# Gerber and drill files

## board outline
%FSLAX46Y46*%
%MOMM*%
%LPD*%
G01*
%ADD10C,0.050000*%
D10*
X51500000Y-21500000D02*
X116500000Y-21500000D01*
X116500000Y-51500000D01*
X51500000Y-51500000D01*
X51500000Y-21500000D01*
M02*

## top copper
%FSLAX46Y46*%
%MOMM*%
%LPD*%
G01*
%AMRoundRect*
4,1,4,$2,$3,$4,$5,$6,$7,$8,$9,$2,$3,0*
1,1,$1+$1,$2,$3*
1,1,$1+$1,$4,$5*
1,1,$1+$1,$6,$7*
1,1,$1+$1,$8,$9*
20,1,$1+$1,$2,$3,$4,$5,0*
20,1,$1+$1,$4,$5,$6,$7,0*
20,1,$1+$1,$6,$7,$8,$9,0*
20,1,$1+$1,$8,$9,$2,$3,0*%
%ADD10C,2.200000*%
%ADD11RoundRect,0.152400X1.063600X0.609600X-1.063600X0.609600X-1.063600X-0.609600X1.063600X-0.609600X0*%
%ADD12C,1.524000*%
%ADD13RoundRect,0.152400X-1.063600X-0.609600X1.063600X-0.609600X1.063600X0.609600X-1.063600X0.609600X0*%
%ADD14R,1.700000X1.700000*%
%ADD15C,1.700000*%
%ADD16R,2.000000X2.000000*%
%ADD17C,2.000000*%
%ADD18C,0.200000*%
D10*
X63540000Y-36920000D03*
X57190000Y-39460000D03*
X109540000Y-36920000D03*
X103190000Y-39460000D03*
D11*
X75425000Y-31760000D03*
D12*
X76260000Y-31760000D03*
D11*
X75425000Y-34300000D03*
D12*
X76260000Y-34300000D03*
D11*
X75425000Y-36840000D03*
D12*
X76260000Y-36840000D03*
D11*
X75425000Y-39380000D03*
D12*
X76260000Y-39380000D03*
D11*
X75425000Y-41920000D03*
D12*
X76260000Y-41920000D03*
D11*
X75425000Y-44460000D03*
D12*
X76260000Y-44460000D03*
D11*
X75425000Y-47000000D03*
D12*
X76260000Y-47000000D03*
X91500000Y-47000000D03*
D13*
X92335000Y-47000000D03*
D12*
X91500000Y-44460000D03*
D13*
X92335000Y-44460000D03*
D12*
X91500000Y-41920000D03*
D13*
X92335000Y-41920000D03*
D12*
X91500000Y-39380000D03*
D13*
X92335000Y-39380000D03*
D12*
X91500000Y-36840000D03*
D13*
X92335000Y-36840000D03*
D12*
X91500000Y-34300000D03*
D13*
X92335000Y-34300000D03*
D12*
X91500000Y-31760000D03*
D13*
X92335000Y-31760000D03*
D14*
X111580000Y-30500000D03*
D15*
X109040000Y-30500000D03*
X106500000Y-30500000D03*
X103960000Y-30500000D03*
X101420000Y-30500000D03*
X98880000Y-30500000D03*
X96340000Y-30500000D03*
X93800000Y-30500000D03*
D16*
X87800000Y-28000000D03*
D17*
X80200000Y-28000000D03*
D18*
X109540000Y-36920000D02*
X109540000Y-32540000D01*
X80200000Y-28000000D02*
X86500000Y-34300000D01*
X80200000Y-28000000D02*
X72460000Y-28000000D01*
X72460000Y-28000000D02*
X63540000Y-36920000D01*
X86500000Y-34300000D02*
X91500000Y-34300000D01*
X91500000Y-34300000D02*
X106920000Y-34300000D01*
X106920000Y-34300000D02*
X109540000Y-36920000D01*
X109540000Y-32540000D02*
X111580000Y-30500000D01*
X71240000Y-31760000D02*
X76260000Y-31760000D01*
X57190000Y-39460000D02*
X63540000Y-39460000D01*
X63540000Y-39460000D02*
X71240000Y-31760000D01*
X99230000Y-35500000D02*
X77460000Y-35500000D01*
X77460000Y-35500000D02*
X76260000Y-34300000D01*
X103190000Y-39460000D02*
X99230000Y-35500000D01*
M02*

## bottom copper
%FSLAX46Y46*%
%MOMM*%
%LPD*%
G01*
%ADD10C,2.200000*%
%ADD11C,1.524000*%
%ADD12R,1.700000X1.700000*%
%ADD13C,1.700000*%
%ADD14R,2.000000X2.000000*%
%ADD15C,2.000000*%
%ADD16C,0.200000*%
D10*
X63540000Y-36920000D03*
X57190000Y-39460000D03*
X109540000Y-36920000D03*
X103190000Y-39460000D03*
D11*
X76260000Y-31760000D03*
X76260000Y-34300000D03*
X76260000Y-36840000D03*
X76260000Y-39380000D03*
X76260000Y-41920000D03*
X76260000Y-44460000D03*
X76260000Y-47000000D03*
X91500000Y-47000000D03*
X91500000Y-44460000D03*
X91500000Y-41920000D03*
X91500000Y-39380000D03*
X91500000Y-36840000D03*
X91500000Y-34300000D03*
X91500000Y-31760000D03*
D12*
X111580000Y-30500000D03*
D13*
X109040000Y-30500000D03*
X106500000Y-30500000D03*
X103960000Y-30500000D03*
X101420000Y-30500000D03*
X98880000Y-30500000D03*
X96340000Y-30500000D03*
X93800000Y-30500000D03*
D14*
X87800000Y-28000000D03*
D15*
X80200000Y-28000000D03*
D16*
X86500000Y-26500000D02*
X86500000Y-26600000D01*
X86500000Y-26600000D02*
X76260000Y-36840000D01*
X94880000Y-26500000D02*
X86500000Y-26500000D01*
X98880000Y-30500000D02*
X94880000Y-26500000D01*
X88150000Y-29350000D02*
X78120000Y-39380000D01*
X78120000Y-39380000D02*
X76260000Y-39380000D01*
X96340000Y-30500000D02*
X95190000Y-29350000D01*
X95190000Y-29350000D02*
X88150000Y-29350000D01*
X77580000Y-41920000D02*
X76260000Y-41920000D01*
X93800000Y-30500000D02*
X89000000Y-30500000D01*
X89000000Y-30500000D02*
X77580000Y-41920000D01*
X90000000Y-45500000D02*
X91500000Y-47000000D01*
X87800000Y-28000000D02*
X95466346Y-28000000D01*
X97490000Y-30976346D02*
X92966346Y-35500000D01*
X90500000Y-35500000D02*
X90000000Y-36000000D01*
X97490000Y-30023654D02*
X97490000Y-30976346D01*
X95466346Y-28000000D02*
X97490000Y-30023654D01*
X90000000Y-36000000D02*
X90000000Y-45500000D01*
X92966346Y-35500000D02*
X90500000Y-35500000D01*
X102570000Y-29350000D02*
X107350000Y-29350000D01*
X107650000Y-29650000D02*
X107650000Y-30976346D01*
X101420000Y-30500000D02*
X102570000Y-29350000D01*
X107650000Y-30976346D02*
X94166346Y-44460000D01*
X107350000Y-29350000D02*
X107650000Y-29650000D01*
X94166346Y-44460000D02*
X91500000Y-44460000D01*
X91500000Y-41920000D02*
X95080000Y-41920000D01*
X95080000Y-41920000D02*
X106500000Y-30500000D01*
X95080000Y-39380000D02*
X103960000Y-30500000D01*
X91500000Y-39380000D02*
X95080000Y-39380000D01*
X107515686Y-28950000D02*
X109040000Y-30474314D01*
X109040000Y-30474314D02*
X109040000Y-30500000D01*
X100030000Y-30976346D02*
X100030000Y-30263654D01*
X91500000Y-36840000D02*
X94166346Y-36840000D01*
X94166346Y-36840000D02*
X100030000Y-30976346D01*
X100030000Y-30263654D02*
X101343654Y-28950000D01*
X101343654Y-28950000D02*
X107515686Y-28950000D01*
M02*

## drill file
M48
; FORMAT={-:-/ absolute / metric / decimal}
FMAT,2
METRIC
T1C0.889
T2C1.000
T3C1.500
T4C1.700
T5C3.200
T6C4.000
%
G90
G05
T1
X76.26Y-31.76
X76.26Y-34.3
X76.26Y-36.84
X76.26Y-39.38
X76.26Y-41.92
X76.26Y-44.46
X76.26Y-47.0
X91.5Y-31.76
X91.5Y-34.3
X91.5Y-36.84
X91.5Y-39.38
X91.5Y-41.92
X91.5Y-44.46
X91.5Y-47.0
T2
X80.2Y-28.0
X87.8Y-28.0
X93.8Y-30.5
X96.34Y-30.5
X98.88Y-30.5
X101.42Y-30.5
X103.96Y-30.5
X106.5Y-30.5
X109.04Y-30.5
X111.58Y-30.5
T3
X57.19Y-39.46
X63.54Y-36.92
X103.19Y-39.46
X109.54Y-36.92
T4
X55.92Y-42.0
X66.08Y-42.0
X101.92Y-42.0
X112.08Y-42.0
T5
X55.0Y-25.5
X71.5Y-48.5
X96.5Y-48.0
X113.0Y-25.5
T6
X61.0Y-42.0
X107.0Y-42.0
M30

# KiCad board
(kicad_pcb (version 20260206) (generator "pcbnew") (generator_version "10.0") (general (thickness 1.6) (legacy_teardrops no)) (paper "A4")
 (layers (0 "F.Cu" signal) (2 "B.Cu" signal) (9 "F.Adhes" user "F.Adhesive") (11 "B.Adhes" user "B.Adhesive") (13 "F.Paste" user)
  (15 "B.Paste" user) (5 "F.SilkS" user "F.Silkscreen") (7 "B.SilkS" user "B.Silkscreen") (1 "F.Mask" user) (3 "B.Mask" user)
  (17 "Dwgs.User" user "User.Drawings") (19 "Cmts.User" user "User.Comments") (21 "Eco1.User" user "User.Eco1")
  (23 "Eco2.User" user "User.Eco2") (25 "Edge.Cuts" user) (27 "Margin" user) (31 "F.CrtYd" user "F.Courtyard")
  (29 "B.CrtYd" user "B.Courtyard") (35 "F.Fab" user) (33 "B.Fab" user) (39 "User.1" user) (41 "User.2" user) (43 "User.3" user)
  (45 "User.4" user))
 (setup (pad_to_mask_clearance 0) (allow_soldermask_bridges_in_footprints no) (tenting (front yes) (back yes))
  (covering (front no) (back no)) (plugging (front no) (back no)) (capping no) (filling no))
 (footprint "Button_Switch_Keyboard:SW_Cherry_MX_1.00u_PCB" (layer "F.Cu") (at 63.54 36.92)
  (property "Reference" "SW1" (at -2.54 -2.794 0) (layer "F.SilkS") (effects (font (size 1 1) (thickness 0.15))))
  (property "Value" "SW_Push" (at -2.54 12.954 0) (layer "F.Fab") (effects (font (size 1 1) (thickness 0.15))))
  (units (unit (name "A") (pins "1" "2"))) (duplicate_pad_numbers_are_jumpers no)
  (pad "" np_thru_hole circle (at -7.62 5.08) (size 1.7 1.7) (drill 1.7) (layers "*.Cu" "*.Mask"))
  (pad "" np_thru_hole circle (at -2.54 5.08) (size 4 4) (drill 4) (layers "*.Cu" "*.Mask"))
  (pad "" np_thru_hole circle (at 2.54 5.08) (size 1.7 1.7) (drill 1.7) (layers "*.Cu" "*.Mask"))
  (pad "1" thru_hole circle (at 0 0) (size 2.2 2.2) (drill 1.5) (layers "*.Cu" "*.Mask") (remove_unused_layers no) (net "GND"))
  (pad "2" thru_hole circle (at -6.35 2.54) (size 2.2 2.2) (drill 1.5) (layers "*.Cu" "*.Mask") (remove_unused_layers no)
   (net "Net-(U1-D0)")))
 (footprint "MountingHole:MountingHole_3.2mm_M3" (layer "F.Cu") (at 96.5 48)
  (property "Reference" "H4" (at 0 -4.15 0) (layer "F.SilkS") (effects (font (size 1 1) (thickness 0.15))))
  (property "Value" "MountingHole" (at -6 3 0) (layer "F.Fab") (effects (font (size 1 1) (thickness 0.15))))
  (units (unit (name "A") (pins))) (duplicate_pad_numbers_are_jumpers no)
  (pad "" np_thru_hole circle (at 0 0) (size 3.2 3.2) (drill 3.2) (layers "*.Cu" "*.Mask")))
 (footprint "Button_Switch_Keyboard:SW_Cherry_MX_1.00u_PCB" (layer "F.Cu") (at 109.54 36.92)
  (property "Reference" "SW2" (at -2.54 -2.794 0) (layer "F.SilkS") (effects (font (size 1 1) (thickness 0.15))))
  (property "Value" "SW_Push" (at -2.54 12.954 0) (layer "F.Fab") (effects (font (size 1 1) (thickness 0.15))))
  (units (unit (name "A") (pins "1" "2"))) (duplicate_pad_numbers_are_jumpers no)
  (pad "" np_thru_hole circle (at -7.62 5.08) (size 1.7 1.7) (drill 1.7) (layers "*.Cu" "*.Mask"))
  (pad "" np_thru_hole circle (at -2.54 5.08) (size 4 4) (drill 4) (layers "*.Cu" "*.Mask"))
  (pad "" np_thru_hole circle (at 2.54 5.08) (size 1.7 1.7) (drill 1.7) (layers "*.Cu" "*.Mask"))
  (pad "1" thru_hole circle (at 0 0) (size 2.2 2.2) (drill 1.5) (layers "*.Cu" "*.Mask") (remove_unused_layers no) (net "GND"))
  (pad "2" thru_hole circle (at -6.35 2.54) (size 2.2 2.2) (drill 1.5) (layers "*.Cu" "*.Mask") (remove_unused_layers no)
   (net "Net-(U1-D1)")))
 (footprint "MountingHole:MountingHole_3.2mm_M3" (layer "F.Cu") (at 71.5 48.5)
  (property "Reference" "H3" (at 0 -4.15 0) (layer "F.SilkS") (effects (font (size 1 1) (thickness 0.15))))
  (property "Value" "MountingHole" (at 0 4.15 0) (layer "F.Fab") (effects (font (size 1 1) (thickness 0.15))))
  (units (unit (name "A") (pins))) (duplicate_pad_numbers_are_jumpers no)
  (pad "" np_thru_hole circle (at 0 0) (size 3.2 3.2) (drill 3.2) (layers "*.Cu" "*.Mask")))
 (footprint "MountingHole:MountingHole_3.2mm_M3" (layer "F.Cu") (at 113 25.5)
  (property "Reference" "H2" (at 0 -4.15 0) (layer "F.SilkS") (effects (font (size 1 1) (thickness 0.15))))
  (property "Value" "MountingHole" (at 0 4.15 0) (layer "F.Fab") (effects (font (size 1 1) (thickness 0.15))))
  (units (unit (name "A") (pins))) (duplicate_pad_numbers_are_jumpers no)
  (pad "" np_thru_hole circle (at 0 0) (size 3.2 3.2) (drill 3.2) (layers "*.Cu" "*.Mask")))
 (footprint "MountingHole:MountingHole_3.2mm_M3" (layer "F.Cu") (at 55 25.5)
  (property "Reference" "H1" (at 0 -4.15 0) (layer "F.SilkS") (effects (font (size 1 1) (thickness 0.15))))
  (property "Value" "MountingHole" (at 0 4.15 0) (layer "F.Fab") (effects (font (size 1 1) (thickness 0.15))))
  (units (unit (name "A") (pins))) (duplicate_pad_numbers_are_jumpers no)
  (pad "" np_thru_hole circle (at 0 0) (size 3.2 3.2) (drill 3.2) (layers "*.Cu" "*.Mask")))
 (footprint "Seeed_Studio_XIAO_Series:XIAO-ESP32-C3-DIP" (layer "F.Cu") (at 83.88 39.38 90)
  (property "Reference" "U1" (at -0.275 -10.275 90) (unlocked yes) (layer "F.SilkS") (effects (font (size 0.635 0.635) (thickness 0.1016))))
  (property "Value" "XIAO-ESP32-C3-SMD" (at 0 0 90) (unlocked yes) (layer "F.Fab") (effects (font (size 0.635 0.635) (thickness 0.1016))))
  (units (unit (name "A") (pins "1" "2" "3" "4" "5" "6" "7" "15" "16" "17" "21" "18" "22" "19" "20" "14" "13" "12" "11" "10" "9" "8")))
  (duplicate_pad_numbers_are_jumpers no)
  (pad "1" smd roundrect (at 7.62 -8.455 180) (size 2.432 1.524) (layers "F.Cu" "F.Mask") (roundrect_rratio 0.1) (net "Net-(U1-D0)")
   (thermal_bridge_angle 45))
  (pad "1" thru_hole circle (at 7.62 -7.62 180) (size 1.524 1.524) (drill 0.889) (layers "*.Cu" "*.Mask") (remove_unused_layers no)
   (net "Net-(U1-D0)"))
  (pad "2" smd roundrect (at 5.08 -8.455 180) (size 2.432 1.524) (layers "F.Cu" "F.Mask") (roundrect_rratio 0.1) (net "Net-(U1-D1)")
   (thermal_bridge_angle 45))
  (pad "2" thru_hole circle (at 5.08 -7.62 180) (size 1.524 1.524) (drill 0.889) (layers "*.Cu" "*.Mask") (remove_unused_layers no)
   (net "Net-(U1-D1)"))
  (pad "3" smd roundrect (at 2.54 -8.455 180) (size 2.432 1.524) (layers "F.Cu" "F.Mask") (roundrect_rratio 0.1) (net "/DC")
   (thermal_bridge_angle 45))
  (pad "3" thru_hole circle (at 2.54 -7.62 180) (size 1.524 1.524) (drill 0.889) (layers "*.Cu" "*.Mask") (remove_unused_layers no)
   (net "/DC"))
  (pad "4" smd roundrect (at 0 -8.455 180) (size 2.432 1.524) (layers "F.Cu" "F.Mask") (roundrect_rratio 0.1) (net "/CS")
   (thermal_bridge_angle 45))
  (pad "4" thru_hole circle (at 0 -7.62 180) (size 1.524 1.524) (drill 0.889) (layers "*.Cu" "*.Mask") (remove_unused_layers no) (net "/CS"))
  (pad "5" smd roundrect (at -2.54 -8.455 180) (size 2.432 1.524) (layers "F.Cu" "F.Mask") (roundrect_rratio 0.1) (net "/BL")
   (thermal_bridge_angle 45))
  (pad "5" thru_hole circle (at -2.54 -7.62 180) (size 1.524 1.524) (drill 0.889) (layers "*.Cu" "*.Mask") (remove_unused_layers no)
   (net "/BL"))
  (pad "6" smd roundrect (at -5.08 -8.455 180) (size 2.432 1.524) (layers "F.Cu" "F.Mask") (roundrect_rratio 0.1)
   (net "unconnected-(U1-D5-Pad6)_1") (thermal_bridge_angle 45))
  (pad "6" thru_hole circle (at -5.08 -7.62 180) (size 1.524 1.524) (drill 0.889) (layers "*.Cu" "*.Mask") (remove_unused_layers no)
   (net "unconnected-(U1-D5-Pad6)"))
  (pad "7" smd roundrect (at -7.62 -8.455 180) (size 2.432 1.524) (layers "F.Cu" "F.Mask") (roundrect_rratio 0.1)
   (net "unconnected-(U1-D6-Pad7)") (thermal_bridge_angle 45))
  (pad "7" thru_hole circle (at -7.62 -7.62 180) (size 1.524 1.524) (drill 0.889) (layers "*.Cu" "*.Mask") (remove_unused_layers no)
   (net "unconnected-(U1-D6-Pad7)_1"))
  (pad "8" thru_hole circle (at -7.62 7.62) (size 1.524 1.524) (drill 0.889) (layers "*.Cu" "*.Mask") (remove_unused_layers no)
   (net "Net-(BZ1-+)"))
  (pad "8" smd roundrect (at -7.62 8.455) (size 2.432 1.524) (layers "F.Cu" "F.Mask") (roundrect_rratio 0.1) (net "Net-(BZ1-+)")
   (thermal_bridge_angle 45))
  (pad "9" thru_hole circle (at -5.08 7.62) (size 1.524 1.524) (drill 0.889) (layers "*.Cu" "*.Mask") (remove_unused_layers no) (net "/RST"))
  (pad "9" smd roundrect (at -5.08 8.455) (size 2.432 1.524) (layers "F.Cu" "F.Mask") (roundrect_rratio 0.1) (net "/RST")
   (thermal_bridge_angle 45))
  (pad "10" thru_hole circle (at -2.54 7.62) (size 1.524 1.524) (drill 0.889) (layers "*.Cu" "*.Mask") (remove_unused_layers no)
   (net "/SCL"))
  (pad "10" smd roundrect (at -2.54 8.455) (size 2.432 1.524) (layers "F.Cu" "F.Mask") (roundrect_rratio 0.1) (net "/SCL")
   (thermal_bridge_angle 45))
  (pad "11" thru_hole circle (at 0 7.62) (size 1.524 1.524) (drill 0.889) (layers "*.Cu" "*.Mask") (remove_unused_layers no) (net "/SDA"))
  (pad "11" smd roundrect (at 0 8.455) (size 2.432 1.524) (layers "F.Cu" "F.Mask") (roundrect_rratio 0.1) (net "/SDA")
   (thermal_bridge_angle 45))
  (pad "12" thru_hole circle (at 2.54 7.62) (size 1.524 1.524) (drill 0.889) (layers "*.Cu" "*.Mask") (remove_unused_layers no)
   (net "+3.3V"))
  (pad "12" smd roundrect (at 2.54 8.455) (size 2.432 1.524) (layers "F.Cu" "F.Mask") (roundrect_rratio 0.1) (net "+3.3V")
   (thermal_bridge_angle 45))
  (pad "13" thru_hole circle (at 5.08 7.62) (size 1.524 1.524) (drill 0.889) (layers "*.Cu" "*.Mask") (remove_unused_layers no) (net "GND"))
  (pad "13" smd roundrect (at 5.08 8.455) (size 2.432 1.524) (layers "F.Cu" "F.Mask") (roundrect_rratio 0.1) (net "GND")
   (thermal_bridge_angle 45))
  (pad "14" thru_hole circle (at 7.62 7.62) (size 1.524 1.524) (drill 0.889) (layers "*.Cu" "*.Mask") (remove_unused_layers no)
   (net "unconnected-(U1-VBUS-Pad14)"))
  (pad "14" smd roundrect (at 7.62 8.455) (size 2.432 1.524) (layers "F.Cu" "F.Mask") (roundrect_rratio 0.1)
   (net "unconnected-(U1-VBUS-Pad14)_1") (thermal_bridge_angle 45)))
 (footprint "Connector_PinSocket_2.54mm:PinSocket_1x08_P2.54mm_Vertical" (layer "B.Cu") (at 111.58 30.5 90)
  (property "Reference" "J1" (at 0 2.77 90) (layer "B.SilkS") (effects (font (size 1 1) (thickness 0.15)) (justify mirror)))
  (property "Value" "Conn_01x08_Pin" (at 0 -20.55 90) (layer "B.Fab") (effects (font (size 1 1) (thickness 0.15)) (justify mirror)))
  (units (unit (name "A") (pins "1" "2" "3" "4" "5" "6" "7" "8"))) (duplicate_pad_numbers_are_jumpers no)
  (pad "1" thru_hole rect (at 0 0 90) (size 1.7 1.7) (drill 1) (layers "*.Cu" "*.Mask") (remove_unused_layers no) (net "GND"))
  (pad "2" thru_hole circle (at 0 -2.54 90) (size 1.7 1.7) (drill 1) (layers "*.Cu" "*.Mask") (remove_unused_layers no) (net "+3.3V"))
  (pad "3" thru_hole circle (at 0 -5.08 90) (size 1.7 1.7) (drill 1) (layers "*.Cu" "*.Mask") (remove_unused_layers no) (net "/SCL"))
  (pad "4" thru_hole circle (at 0 -7.62 90) (size 1.7 1.7) (drill 1) (layers "*.Cu" "*.Mask") (remove_unused_layers no) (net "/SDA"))
  (pad "5" thru_hole circle (at 0 -10.16 90) (size 1.7 1.7) (drill 1) (layers "*.Cu" "*.Mask") (remove_unused_layers no) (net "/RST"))
  (pad "6" thru_hole circle (at 0 -12.7 90) (size 1.7 1.7) (drill 1) (layers "*.Cu" "*.Mask") (remove_unused_layers no) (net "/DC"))
  (pad "7" thru_hole circle (at 0 -15.24 90) (size 1.7 1.7) (drill 1) (layers "*.Cu" "*.Mask") (remove_unused_layers no) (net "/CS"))
  (pad "8" thru_hole circle (at 0 -17.78 90) (size 1.7 1.7) (drill 1) (layers "*.Cu" "*.Mask") (remove_unused_layers no) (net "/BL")))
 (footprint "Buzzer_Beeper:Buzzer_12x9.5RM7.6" (layer "B.Cu") (at 87.8 28 180)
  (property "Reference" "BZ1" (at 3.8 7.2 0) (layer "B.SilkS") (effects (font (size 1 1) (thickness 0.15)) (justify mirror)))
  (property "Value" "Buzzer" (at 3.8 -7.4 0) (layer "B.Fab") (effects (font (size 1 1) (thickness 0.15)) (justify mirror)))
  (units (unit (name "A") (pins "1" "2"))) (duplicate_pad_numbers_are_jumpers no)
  (pad "1" thru_hole rect (at 0 0 180) (size 2 2) (drill 1) (layers "*.Cu" "*.Mask") (remove_unused_layers no) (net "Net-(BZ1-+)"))
  (pad "2" thru_hole circle (at 7.6 0 180) (size 2 2) (drill 1) (layers "*.Cu" "*.Mask") (remove_unused_layers no) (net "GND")))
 (gr_rect (start 51.5 21.5) (end 116.5 51.5) (stroke (width 0.05) (type default)) (fill no) (layer "Edge.Cuts"))
 (segment (start 109.54 36.92) (end 109.54 32.54) (width 0.2) (layer "F.Cu") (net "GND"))
 (segment (start 80.2 28) (end 86.5 34.3) (width 0.2) (layer "F.Cu") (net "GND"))
 (segment (start 80.2 28) (end 72.46 28) (width 0.2) (layer "F.Cu") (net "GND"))
 (segment (start 72.46 28) (end 63.54 36.92) (width 0.2) (layer "F.Cu") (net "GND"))
 (segment (start 86.5 34.3) (end 91.5 34.3) (width 0.2) (layer "F.Cu") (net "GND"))
 (segment (start 91.5 34.3) (end 106.92 34.3) (width 0.2) (layer "F.Cu") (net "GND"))
 (segment (start 106.92 34.3) (end 109.54 36.92) (width 0.2) (layer "F.Cu") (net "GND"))
 (segment (start 109.54 32.54) (end 111.58 30.5) (width 0.2) (layer "F.Cu") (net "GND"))
 (segment (start 71.24 31.76) (end 76.26 31.76) (width 0.2) (layer "F.Cu") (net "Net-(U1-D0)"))
 (segment (start 57.19 39.46) (end 63.54 39.46) (width 0.2) (layer "F.Cu") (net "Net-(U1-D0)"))
 (segment (start 63.54 39.46) (end 71.24 31.76) (width 0.2) (layer "F.Cu") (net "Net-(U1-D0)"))
 (segment (start 99.23 35.5) (end 77.46 35.5) (width 0.2) (layer "F.Cu") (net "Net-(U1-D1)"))
 (segment (start 77.46 35.5) (end 76.26 34.3) (width 0.2) (layer "F.Cu") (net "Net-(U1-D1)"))
 (segment (start 103.19 39.46) (end 99.23 35.5) (width 0.2) (layer "F.Cu") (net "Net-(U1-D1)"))
 (segment (start 86.5 26.5) (end 86.5 26.6) (width 0.2) (layer "B.Cu") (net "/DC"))
 (segment (start 86.5 26.6) (end 76.26 36.84) (width 0.2) (layer "B.Cu") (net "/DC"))
 (segment (start 94.88 26.5) (end 86.5 26.5) (width 0.2) (layer "B.Cu") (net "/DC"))
 (segment (start 98.88 30.5) (end 94.88 26.5) (width 0.2) (layer "B.Cu") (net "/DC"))
 (segment (start 88.15 29.35) (end 78.12 39.38) (width 0.2) (layer "B.Cu") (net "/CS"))
 (segment (start 78.12 39.38) (end 76.26 39.38) (width 0.2) (layer "B.Cu") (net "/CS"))
 (segment (start 96.34 30.5) (end 95.19 29.35) (width 0.2) (layer "B.Cu") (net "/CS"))
 (segment (start 95.19 29.35) (end 88.15 29.35) (width 0.2) (layer "B.Cu") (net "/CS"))
 (segment (start 77.58 41.92) (end 76.26 41.92) (width 0.2) (layer "B.Cu") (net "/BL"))
 (segment (start 93.8 30.5) (end 89 30.5) (width 0.2) (layer "B.Cu") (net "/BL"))
 (segment (start 89 30.5) (end 77.58 41.92) (width 0.2) (layer "B.Cu") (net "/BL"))
 (segment (start 90 45.5) (end 91.5 47) (width 0.2) (layer "B.Cu") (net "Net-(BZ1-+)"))
 (segment (start 87.8 28) (end 95.466346 28) (width 0.2) (layer "B.Cu") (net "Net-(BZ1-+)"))
 (segment (start 97.49 30.976346) (end 92.966346 35.5) (width 0.2) (layer "B.Cu") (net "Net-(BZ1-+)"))
 (segment (start 90.5 35.5) (end 90 36) (width 0.2) (layer "B.Cu") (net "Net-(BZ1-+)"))
 (segment (start 97.49 30.023654) (end 97.49 30.976346) (width 0.2) (layer "B.Cu") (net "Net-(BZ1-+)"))
 (segment (start 95.466346 28) (end 97.49 30.023654) (width 0.2) (layer "B.Cu") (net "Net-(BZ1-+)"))
 (segment (start 90 36) (end 90 45.5) (width 0.2) (layer "B.Cu") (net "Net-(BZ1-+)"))
 (segment (start 92.966346 35.5) (end 90.5 35.5) (width 0.2) (layer "B.Cu") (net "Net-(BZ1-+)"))
 (segment (start 102.57 29.35) (end 107.35 29.35) (width 0.2) (layer "B.Cu") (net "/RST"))
 (segment (start 107.65 29.65) (end 107.65 30.976346) (width 0.2) (layer "B.Cu") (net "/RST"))
 (segment (start 101.42 30.5) (end 102.57 29.35) (width 0.2) (layer "B.Cu") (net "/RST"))
 (segment (start 107.65 30.976346) (end 94.166346 44.46) (width 0.2) (layer "B.Cu") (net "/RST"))
 (segment (start 107.35 29.35) (end 107.65 29.65) (width 0.2) (layer "B.Cu") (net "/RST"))
 (segment (start 94.166346 44.46) (end 91.5 44.46) (width 0.2) (layer "B.Cu") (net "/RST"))
 (segment (start 91.5 41.92) (end 95.08 41.92) (width 0.2) (layer "B.Cu") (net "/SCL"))
 (segment (start 95.08 41.92) (end 106.5 30.5) (width 0.2) (layer "B.Cu") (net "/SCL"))
 (segment (start 95.08 39.38) (end 103.96 30.5) (width 0.2) (layer "B.Cu") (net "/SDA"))
 (segment (start 91.5 39.38) (end 95.08 39.38) (width 0.2) (layer "B.Cu") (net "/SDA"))
 (segment (start 107.515686 28.95) (end 109.04 30.474314) (width 0.2) (layer "B.Cu") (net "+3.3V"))
 (segment (start 109.04 30.474314) (end 109.04 30.5) (width 0.2) (layer "B.Cu") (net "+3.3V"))
 (segment (start 100.03 30.976346) (end 100.03 30.263654) (width 0.2) (layer "B.Cu") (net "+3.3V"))
 (segment (start 91.5 36.84) (end 94.166346 36.84) (width 0.2) (layer "B.Cu") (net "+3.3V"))
 (segment (start 94.166346 36.84) (end 100.03 30.976346) (width 0.2) (layer "B.Cu") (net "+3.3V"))
 (segment (start 100.03 30.263654) (end 101.343654 28.95) (width 0.2) (layer "B.Cu") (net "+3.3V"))
 (segment (start 101.343654 28.95) (end 107.515686 28.95) (width 0.2) (layer "B.Cu") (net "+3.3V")))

